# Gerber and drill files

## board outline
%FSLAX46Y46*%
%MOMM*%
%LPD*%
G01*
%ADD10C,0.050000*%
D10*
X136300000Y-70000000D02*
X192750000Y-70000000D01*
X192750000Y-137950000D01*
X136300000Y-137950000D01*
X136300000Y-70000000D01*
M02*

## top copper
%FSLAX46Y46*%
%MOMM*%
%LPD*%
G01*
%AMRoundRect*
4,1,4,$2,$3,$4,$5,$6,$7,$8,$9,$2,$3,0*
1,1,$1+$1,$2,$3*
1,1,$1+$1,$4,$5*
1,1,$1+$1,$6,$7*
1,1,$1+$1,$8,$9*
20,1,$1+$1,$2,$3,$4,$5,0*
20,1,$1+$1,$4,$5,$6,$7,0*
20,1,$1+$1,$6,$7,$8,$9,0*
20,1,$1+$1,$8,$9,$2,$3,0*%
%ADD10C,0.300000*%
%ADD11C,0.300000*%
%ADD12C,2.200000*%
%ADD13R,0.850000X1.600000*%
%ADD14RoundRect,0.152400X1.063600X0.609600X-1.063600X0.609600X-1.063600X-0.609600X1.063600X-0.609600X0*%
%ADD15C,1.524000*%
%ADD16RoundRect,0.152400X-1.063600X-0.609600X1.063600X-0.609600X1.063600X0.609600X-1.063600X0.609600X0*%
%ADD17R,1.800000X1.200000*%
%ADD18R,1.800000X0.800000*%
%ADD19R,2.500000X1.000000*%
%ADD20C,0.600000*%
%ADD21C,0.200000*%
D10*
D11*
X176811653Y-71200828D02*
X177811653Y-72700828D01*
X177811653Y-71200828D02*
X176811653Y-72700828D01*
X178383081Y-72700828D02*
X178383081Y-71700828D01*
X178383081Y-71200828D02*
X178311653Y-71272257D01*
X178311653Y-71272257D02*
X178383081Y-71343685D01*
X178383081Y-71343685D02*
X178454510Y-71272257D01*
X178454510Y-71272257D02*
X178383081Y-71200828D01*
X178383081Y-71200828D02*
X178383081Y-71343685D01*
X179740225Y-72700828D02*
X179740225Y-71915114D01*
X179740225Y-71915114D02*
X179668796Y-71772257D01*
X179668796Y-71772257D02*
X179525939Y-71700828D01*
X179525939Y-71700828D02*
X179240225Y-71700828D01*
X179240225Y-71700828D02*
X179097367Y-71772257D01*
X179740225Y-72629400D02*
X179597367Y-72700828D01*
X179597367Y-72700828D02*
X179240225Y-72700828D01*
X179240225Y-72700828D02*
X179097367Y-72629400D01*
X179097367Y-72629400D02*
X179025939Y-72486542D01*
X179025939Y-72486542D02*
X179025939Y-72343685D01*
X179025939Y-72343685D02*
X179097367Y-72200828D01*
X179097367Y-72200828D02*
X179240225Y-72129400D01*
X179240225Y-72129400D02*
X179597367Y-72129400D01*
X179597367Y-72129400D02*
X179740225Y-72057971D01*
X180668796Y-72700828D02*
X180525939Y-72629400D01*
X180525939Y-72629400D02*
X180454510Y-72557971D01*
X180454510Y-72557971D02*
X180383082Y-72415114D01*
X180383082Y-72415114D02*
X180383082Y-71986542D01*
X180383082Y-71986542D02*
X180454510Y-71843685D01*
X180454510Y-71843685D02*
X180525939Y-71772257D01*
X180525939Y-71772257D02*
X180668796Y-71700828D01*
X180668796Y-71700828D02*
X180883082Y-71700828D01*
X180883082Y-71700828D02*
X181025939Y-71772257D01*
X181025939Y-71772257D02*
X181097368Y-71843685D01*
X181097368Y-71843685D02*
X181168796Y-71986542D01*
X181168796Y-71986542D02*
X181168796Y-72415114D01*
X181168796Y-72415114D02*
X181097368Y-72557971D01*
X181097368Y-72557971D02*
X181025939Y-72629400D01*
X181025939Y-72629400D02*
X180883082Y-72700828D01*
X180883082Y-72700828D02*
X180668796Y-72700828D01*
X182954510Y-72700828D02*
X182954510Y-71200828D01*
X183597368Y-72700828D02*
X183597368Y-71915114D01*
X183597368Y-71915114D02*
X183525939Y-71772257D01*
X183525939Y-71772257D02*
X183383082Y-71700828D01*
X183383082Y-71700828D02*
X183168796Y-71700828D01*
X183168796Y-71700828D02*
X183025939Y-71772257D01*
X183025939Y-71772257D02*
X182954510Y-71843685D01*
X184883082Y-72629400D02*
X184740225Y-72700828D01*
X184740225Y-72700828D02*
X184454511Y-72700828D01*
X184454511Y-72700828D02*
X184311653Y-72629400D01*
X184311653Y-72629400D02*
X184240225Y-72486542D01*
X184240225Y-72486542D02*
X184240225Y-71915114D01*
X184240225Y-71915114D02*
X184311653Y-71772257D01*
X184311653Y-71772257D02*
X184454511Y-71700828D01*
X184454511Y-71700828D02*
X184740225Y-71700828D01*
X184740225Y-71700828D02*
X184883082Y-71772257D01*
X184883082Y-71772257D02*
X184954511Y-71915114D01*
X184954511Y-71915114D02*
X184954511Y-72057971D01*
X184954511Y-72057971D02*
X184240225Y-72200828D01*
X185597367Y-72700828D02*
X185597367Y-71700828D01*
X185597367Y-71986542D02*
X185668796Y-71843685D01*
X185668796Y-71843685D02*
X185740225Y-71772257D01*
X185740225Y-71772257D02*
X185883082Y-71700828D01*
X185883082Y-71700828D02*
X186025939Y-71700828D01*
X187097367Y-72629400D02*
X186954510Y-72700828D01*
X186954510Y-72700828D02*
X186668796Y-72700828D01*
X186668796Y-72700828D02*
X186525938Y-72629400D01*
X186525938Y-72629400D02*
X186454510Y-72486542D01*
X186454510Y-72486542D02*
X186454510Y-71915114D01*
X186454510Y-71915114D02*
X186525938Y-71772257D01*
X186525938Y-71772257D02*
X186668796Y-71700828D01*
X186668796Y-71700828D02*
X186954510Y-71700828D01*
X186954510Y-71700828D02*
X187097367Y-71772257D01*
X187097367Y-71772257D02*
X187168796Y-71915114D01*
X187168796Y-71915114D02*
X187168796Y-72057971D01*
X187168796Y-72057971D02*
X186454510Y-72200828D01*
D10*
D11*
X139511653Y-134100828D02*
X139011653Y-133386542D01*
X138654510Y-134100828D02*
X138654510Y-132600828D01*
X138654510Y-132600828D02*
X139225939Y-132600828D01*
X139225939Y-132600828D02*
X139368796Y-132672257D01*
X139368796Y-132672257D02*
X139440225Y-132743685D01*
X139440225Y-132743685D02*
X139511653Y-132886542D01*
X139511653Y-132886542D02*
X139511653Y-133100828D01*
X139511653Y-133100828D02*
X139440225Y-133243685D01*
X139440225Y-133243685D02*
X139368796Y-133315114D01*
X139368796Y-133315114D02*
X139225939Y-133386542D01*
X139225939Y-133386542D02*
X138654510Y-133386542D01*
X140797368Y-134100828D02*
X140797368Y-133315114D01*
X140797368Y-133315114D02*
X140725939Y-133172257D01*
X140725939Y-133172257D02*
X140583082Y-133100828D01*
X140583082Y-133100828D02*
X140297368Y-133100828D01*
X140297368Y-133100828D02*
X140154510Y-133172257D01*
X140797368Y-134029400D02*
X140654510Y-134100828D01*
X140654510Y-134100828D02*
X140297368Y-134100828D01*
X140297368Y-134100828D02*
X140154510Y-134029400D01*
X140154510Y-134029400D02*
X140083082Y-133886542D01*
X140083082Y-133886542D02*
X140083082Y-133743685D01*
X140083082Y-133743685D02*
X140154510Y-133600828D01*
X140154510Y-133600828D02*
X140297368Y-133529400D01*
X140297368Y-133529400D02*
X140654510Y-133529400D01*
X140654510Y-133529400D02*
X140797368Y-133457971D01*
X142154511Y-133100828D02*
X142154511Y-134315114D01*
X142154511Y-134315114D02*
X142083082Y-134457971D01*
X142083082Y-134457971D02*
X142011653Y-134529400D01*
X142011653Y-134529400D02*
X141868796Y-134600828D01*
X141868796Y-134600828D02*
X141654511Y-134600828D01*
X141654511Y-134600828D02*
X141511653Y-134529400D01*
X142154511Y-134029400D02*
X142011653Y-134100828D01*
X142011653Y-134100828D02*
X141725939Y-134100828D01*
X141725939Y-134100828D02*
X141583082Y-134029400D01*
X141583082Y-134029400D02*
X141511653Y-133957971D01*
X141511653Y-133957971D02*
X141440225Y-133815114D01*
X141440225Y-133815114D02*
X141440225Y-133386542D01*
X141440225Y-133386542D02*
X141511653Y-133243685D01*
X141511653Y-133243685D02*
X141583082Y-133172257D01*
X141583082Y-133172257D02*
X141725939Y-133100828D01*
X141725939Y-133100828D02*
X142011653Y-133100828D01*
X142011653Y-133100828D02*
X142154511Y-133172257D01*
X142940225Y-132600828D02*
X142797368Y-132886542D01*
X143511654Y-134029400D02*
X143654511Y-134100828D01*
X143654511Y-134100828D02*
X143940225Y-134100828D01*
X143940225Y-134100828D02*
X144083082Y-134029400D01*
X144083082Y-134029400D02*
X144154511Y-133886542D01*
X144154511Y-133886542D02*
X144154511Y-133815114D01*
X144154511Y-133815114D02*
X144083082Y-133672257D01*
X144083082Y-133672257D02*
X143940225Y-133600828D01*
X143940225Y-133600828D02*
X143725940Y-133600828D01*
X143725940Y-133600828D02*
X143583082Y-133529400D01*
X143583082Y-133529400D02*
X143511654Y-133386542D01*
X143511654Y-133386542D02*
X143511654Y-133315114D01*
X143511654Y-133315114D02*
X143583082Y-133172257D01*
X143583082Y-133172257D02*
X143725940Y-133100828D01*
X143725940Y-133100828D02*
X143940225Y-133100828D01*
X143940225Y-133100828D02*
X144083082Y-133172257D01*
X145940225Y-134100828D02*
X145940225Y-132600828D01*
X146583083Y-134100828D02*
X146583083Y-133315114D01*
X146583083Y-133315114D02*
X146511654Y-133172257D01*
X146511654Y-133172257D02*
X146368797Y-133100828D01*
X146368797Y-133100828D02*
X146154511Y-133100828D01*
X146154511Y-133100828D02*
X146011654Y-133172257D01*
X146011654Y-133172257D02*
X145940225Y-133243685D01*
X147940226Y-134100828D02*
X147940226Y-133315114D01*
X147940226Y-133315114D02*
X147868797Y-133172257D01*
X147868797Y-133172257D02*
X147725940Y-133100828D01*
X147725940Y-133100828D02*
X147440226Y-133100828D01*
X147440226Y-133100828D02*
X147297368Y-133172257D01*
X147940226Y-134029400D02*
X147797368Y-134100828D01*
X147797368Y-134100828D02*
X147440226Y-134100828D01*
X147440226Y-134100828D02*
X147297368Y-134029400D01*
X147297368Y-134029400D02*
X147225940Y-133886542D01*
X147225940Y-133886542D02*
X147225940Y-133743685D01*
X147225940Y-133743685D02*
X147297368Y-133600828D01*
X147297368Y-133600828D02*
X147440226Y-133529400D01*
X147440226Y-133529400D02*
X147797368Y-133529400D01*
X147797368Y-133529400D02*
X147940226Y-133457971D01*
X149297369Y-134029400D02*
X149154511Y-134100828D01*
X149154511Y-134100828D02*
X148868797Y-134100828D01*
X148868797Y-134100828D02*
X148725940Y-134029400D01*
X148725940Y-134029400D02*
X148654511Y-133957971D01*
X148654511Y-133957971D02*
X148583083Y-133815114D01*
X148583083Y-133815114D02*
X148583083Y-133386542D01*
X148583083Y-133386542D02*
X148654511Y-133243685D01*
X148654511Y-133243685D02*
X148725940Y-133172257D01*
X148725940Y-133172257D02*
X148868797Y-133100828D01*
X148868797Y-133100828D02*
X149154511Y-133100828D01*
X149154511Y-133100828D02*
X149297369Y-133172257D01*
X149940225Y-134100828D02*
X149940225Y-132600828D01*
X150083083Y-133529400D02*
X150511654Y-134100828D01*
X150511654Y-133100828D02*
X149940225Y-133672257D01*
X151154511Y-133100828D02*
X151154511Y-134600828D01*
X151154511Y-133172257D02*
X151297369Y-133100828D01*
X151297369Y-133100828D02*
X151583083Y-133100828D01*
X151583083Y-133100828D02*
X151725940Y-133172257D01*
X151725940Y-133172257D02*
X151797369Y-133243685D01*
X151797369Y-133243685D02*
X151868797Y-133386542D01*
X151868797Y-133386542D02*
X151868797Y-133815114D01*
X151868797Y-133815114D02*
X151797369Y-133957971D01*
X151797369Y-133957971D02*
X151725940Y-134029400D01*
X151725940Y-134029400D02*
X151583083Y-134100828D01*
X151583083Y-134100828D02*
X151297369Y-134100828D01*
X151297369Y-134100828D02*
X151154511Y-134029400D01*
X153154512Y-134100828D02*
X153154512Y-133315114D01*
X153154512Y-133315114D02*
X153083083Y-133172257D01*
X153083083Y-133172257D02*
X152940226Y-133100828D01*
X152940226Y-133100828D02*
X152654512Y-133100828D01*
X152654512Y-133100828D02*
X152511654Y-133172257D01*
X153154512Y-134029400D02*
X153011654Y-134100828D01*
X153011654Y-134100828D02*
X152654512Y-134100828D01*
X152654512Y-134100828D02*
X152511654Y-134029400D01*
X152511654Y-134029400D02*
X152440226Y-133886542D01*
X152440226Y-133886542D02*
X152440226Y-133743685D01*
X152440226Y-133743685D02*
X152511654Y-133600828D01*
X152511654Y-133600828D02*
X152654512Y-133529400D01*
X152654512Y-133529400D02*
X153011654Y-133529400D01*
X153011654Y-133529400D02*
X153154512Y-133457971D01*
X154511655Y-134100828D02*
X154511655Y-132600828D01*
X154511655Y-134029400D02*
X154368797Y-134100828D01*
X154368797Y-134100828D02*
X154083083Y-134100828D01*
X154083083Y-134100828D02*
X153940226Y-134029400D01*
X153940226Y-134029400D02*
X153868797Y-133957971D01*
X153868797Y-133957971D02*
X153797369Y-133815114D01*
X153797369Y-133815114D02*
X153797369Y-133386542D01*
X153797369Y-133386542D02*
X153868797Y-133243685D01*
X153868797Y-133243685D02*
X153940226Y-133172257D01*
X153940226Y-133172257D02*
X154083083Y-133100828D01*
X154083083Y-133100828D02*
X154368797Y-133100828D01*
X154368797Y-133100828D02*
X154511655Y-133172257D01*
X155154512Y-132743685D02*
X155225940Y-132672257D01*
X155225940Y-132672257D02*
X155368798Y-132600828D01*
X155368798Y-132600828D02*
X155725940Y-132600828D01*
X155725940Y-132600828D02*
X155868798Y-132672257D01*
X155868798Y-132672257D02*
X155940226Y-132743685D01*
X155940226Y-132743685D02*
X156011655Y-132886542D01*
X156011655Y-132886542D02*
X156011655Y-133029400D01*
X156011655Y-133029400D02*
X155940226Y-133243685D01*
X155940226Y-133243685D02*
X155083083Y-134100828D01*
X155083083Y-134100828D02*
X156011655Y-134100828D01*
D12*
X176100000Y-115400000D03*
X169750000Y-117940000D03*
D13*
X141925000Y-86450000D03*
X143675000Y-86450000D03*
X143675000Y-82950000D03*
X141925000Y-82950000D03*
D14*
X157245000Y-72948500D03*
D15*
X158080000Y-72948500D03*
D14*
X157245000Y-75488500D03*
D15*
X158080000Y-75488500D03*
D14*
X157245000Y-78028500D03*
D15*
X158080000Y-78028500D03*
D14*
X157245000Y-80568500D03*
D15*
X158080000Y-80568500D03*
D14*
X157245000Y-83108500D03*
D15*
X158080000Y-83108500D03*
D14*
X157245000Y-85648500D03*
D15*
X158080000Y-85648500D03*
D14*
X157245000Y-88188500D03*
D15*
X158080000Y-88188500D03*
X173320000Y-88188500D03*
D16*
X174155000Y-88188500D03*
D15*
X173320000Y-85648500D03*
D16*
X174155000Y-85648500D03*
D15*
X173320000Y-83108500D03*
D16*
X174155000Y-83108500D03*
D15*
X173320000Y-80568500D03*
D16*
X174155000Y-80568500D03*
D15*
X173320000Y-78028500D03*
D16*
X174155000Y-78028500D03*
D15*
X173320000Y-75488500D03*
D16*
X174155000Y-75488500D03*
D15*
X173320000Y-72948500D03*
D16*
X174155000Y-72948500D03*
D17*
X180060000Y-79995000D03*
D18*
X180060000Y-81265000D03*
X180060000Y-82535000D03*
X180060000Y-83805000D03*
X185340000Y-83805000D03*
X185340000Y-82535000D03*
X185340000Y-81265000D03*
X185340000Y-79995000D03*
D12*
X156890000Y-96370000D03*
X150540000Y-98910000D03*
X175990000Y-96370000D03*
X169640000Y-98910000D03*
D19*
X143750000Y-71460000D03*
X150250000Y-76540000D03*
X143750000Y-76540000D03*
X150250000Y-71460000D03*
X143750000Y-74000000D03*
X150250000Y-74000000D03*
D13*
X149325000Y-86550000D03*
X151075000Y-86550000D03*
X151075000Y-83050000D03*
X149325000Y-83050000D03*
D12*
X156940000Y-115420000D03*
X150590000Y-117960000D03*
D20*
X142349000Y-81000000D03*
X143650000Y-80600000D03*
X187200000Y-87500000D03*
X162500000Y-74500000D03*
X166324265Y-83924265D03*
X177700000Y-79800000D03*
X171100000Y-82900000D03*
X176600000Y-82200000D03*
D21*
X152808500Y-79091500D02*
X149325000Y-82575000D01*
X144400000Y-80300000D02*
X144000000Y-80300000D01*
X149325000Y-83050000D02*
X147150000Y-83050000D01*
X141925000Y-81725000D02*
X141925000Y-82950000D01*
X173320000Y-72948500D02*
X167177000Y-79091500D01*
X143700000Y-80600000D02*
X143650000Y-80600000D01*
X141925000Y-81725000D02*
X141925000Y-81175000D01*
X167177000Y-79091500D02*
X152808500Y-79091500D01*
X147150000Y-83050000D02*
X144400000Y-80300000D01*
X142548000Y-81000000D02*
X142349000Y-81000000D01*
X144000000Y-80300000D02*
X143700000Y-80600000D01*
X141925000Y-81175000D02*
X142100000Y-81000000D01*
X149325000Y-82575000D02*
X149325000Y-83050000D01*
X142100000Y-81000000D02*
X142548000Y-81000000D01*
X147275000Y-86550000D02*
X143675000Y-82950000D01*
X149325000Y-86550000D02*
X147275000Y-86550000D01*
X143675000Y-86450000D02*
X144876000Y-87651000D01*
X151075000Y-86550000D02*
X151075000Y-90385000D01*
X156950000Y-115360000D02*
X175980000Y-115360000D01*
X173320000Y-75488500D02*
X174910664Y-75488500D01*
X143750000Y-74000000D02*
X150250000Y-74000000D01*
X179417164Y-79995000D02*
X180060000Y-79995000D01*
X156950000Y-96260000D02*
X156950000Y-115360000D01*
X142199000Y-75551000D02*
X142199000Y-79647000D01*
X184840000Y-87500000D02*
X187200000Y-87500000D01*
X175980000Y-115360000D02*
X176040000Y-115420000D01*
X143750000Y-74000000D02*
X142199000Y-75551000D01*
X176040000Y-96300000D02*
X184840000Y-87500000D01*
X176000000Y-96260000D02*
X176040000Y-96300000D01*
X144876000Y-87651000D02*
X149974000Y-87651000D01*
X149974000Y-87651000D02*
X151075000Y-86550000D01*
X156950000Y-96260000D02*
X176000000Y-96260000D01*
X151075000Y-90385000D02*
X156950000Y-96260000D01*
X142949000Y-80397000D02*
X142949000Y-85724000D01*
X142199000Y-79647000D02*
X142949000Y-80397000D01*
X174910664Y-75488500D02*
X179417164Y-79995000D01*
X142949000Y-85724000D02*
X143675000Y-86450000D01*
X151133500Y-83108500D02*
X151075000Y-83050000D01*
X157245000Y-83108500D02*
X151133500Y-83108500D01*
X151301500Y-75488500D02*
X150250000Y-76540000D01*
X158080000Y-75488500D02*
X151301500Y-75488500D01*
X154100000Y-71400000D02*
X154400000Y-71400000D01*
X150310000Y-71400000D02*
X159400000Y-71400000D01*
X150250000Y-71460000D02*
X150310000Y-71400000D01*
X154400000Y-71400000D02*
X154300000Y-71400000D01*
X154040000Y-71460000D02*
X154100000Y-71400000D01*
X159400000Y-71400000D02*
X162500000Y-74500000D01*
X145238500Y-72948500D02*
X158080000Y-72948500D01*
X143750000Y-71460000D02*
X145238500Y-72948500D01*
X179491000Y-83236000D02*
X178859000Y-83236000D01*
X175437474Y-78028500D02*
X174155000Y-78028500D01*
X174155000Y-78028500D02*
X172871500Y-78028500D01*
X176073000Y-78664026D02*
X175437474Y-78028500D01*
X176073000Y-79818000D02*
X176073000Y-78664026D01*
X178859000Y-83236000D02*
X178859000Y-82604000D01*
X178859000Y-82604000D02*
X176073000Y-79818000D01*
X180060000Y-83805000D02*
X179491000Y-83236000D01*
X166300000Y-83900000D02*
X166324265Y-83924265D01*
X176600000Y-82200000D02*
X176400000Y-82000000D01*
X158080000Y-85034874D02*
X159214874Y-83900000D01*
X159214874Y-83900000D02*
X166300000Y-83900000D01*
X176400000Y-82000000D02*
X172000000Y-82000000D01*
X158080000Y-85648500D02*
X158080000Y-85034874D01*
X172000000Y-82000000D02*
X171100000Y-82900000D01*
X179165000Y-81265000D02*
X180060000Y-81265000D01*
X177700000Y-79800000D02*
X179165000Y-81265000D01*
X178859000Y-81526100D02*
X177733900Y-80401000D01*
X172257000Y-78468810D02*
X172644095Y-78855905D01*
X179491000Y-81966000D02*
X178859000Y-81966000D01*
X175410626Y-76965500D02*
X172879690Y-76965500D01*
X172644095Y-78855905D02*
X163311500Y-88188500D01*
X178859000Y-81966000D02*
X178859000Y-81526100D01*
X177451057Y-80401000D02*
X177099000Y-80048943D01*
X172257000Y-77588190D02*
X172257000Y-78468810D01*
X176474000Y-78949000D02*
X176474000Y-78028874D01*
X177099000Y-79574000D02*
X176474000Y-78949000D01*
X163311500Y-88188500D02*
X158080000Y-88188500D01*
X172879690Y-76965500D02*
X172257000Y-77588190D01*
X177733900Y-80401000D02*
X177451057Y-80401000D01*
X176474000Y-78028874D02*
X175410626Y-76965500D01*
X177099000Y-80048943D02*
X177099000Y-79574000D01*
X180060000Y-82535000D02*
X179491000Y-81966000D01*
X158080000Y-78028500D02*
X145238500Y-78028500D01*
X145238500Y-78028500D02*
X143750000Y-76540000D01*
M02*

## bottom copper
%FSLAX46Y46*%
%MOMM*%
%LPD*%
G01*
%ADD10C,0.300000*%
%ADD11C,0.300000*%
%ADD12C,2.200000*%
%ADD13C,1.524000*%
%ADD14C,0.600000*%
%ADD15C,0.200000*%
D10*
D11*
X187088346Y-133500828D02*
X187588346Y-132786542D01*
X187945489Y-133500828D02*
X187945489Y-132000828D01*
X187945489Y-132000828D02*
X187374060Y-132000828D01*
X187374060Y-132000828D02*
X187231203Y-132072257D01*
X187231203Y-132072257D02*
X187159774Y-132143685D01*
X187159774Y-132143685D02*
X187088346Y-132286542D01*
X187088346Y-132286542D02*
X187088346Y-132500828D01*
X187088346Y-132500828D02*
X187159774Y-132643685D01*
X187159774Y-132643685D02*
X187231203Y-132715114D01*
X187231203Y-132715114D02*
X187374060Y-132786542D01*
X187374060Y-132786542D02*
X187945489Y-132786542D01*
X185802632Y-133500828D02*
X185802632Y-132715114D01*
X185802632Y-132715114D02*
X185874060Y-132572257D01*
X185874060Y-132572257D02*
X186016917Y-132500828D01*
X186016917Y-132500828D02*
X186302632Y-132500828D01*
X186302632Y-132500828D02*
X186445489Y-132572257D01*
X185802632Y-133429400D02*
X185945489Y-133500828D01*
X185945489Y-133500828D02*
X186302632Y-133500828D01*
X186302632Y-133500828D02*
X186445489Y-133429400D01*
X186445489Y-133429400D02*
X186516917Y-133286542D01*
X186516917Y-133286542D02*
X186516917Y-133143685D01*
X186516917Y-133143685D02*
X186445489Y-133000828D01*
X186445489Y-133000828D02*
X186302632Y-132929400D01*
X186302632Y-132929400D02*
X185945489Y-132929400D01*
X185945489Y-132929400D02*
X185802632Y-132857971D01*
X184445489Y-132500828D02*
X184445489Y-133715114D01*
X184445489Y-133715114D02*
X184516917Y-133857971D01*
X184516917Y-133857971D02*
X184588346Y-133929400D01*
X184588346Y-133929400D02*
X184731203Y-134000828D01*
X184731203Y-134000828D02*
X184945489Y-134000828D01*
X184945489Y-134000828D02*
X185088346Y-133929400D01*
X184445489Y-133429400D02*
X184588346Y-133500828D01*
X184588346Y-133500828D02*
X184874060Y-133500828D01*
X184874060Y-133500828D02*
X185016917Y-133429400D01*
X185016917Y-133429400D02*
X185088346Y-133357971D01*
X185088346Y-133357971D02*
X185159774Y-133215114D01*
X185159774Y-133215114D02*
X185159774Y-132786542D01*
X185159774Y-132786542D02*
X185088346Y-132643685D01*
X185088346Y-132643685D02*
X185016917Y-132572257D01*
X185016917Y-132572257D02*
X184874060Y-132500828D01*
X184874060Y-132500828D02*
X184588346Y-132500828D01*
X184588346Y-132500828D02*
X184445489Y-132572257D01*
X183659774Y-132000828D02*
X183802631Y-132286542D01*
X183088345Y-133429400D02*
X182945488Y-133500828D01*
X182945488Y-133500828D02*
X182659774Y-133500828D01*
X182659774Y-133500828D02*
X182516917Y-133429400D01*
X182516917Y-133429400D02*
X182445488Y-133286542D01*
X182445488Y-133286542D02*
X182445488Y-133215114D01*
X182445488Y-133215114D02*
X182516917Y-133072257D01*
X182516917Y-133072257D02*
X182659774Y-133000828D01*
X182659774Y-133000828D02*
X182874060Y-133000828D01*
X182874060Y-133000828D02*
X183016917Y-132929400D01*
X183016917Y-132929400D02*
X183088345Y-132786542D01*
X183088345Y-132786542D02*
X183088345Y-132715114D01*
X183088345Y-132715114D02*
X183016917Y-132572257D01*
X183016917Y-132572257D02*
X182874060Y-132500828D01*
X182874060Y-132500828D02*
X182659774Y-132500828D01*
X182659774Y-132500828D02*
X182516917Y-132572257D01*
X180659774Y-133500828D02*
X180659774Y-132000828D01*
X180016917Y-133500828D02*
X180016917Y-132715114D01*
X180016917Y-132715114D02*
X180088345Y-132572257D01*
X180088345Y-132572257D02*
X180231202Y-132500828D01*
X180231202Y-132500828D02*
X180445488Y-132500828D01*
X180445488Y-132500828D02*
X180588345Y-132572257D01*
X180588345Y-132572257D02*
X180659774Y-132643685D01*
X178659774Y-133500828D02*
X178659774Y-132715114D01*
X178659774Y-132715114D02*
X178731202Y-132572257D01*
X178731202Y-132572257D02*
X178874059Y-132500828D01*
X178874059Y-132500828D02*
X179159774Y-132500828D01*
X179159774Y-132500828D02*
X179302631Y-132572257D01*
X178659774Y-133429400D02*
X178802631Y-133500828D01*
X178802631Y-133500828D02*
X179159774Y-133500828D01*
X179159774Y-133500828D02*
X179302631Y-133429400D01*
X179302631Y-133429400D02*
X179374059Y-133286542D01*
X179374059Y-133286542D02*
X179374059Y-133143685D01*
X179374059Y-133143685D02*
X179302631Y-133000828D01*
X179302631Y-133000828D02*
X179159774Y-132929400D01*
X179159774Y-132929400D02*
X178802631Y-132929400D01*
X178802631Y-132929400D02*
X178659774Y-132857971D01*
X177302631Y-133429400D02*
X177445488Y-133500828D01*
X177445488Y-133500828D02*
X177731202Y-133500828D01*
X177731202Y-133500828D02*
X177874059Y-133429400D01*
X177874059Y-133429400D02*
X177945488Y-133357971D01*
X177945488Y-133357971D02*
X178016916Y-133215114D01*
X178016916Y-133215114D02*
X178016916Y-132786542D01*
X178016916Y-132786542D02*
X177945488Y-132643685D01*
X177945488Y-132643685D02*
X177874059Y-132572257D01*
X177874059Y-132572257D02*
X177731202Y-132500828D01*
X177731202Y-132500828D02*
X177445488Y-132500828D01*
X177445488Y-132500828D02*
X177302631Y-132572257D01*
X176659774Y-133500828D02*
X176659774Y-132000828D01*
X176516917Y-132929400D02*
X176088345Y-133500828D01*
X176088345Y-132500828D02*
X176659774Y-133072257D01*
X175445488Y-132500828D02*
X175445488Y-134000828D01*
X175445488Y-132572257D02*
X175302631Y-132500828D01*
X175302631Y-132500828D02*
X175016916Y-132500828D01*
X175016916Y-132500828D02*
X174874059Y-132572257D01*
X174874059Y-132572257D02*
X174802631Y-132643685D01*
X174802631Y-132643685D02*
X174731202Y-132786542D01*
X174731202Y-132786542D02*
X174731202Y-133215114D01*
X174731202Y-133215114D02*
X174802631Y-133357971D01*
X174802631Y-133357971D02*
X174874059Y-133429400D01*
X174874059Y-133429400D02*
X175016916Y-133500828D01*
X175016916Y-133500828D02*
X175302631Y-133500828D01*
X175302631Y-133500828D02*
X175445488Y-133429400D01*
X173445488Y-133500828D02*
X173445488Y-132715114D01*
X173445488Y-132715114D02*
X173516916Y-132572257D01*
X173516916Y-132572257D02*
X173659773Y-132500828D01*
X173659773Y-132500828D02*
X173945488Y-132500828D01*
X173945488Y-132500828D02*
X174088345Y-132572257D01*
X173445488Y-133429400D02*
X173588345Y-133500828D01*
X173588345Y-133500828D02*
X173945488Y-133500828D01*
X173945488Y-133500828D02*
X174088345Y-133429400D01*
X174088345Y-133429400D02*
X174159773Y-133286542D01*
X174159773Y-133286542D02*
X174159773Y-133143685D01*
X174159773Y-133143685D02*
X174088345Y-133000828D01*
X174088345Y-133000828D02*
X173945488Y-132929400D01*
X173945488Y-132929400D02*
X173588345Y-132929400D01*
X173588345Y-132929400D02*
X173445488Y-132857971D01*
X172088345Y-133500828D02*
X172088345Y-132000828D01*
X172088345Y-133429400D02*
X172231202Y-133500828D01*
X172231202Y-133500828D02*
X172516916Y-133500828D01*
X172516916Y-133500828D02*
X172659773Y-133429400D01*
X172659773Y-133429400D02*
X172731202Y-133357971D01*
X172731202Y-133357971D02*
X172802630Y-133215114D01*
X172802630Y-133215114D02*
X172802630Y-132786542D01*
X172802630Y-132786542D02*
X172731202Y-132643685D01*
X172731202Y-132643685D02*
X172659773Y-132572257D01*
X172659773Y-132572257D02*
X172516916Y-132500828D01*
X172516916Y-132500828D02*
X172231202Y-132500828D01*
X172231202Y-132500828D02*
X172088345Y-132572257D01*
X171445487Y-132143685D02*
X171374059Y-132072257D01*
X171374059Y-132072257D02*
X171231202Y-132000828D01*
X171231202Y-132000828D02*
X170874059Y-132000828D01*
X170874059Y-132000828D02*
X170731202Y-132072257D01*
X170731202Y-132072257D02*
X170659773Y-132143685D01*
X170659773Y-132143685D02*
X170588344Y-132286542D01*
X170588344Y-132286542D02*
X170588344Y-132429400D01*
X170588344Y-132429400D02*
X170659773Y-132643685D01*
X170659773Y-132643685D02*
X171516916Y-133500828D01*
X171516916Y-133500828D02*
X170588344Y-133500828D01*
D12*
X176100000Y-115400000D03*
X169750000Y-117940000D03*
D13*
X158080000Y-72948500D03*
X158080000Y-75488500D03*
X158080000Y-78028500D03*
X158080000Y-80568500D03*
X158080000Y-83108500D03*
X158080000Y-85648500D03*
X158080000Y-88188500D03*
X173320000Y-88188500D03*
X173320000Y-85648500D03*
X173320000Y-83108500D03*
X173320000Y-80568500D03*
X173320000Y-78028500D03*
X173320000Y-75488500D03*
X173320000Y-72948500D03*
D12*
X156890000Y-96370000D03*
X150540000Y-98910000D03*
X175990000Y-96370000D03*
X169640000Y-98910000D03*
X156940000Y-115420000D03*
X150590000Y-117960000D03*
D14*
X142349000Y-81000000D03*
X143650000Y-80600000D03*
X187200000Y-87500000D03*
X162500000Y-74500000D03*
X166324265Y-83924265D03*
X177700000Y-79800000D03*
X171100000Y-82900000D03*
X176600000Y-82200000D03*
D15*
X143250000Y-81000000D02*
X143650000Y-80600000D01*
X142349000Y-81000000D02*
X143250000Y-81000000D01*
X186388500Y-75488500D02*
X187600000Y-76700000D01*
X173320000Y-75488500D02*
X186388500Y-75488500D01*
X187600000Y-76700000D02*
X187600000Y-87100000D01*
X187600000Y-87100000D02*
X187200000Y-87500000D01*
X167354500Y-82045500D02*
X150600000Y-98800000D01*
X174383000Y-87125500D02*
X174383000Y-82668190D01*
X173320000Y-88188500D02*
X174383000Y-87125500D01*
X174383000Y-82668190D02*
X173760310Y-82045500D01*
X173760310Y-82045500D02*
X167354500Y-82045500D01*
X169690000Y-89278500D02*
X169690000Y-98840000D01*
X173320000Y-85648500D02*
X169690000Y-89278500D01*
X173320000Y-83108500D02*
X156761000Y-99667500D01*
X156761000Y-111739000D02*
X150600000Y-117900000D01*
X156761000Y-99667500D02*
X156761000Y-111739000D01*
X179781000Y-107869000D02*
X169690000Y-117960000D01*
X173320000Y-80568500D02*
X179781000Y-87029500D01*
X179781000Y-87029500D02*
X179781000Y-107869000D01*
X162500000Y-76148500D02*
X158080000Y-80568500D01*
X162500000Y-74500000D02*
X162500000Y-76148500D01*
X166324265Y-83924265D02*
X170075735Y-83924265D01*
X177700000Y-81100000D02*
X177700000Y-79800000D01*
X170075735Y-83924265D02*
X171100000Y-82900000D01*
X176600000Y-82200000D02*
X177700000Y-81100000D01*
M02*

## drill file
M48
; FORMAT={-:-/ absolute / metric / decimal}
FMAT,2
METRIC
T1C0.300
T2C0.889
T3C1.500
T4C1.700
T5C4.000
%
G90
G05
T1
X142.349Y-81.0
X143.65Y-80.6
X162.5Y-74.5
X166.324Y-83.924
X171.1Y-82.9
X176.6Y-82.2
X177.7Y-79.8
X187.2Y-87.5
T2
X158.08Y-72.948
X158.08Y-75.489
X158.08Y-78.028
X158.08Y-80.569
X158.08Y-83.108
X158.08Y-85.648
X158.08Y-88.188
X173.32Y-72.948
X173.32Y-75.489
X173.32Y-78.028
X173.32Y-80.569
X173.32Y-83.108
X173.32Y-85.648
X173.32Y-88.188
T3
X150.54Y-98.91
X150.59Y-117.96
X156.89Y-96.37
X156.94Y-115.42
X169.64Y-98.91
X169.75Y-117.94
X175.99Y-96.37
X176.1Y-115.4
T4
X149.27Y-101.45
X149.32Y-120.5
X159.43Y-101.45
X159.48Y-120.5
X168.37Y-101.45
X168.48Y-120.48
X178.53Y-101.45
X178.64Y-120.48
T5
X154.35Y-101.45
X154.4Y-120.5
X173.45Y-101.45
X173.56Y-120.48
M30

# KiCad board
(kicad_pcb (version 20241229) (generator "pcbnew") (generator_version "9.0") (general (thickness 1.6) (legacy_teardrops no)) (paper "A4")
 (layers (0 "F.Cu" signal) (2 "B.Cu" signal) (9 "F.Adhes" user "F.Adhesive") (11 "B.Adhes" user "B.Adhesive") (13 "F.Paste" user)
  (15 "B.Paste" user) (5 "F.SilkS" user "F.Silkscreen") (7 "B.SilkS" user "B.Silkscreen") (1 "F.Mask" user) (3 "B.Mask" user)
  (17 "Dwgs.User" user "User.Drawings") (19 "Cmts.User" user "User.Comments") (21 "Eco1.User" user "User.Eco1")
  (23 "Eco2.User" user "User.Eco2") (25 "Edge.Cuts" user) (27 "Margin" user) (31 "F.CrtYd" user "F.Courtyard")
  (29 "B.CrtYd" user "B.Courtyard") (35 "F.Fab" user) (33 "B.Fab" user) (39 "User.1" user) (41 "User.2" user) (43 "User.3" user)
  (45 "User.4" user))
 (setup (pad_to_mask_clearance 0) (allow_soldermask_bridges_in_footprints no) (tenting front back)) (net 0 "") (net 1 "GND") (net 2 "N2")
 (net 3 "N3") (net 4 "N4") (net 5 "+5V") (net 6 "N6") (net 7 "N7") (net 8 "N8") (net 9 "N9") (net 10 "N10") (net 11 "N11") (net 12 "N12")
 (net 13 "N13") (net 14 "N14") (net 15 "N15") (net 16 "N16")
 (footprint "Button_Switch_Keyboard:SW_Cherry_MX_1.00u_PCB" (layer "F.Cu") (at 176.1 115.4)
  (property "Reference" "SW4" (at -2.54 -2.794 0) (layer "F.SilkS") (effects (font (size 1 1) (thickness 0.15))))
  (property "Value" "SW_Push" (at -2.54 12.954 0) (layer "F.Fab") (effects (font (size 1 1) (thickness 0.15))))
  (pad "" np_thru_hole circle (at -7.62 5.08) (size 1.7 1.7) (drill 1.7) (layers "*.Cu" "*.Mask"))
  (pad "" np_thru_hole circle (at -2.54 5.08) (size 4 4) (drill 4) (layers "*.Cu" "*.Mask"))
  (pad "" np_thru_hole circle (at 2.54 5.08) (size 1.7 1.7) (drill 1.7) (layers "*.Cu" "*.Mask"))
  (pad "1" thru_hole circle (at 0 0) (size 2.2 2.2) (drill 1.5) (layers "*.Cu" "*.Mask") (remove_unused_layers no) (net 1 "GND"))
  (pad "2" thru_hole circle (at -6.35 2.54) (size 2.2 2.2) (drill 1.5) (layers "*.Cu" "*.Mask") (remove_unused_layers no) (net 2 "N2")))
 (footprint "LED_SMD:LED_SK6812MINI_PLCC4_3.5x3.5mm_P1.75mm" (layer "F.Cu") (at 142.8 84.7 90)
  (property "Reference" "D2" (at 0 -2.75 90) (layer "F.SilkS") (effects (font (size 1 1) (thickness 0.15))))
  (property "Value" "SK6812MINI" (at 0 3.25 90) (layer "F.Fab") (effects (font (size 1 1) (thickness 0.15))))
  (pad "1" smd rect (at -1.75 -0.875 90) (size 1.6 0.85) (layers "F.Cu" "F.Mask" "F.Paste") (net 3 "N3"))
  (pad "2" smd rect (at -1.75 0.875 90) (size 1.6 0.85) (layers "F.Cu" "F.Mask" "F.Paste") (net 1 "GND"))
  (pad "3" smd rect (at 1.75 0.875 90) (size 1.6 0.85) (layers "F.Cu" "F.Mask" "F.Paste") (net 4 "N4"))
  (pad "4" smd rect (at 1.75 -0.875 90) (size 1.6 0.85) (layers "F.Cu" "F.Mask" "F.Paste") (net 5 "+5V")))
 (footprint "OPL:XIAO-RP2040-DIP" (layer "F.Cu") (at 165.7 80.5685)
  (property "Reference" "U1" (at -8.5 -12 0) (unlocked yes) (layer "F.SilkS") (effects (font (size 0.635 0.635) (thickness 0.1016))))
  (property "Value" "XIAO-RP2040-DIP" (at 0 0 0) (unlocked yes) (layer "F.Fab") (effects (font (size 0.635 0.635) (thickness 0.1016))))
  (pad "1" smd roundrect (at -8.455 -7.62 180) (size 2.432 1.524) (layers "F.Cu" "F.Mask") (roundrect_rratio 0.1) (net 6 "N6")
   (thermal_bridge_angle 45))
  (pad "1" thru_hole circle (at -7.62 -7.62 180) (size 1.524 1.524) (drill 0.889) (layers "*.Cu" "*.Mask") (remove_unused_layers no)
   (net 6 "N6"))
  (pad "2" smd roundrect (at -8.455 -5.08 180) (size 2.432 1.524) (layers "F.Cu" "F.Mask") (roundrect_rratio 0.1) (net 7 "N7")
   (thermal_bridge_angle 45))
  (pad "2" thru_hole circle (at -7.62 -5.08 180) (size 1.524 1.524) (drill 0.889) (layers "*.Cu" "*.Mask") (remove_unused_layers no)
   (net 7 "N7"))
  (pad "3" smd roundrect (at -8.455 -2.54 180) (size 2.432 1.524) (layers "F.Cu" "F.Mask") (roundrect_rratio 0.1) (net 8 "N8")
   (thermal_bridge_angle 45))
  (pad "3" thru_hole circle (at -7.62 -2.54 180) (size 1.524 1.524) (drill 0.889) (layers "*.Cu" "*.Mask") (remove_unused_layers no)
   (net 8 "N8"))
  (pad "4" smd roundrect (at -8.455 0 180) (size 2.432 1.524) (layers "F.Cu" "F.Mask") (roundrect_rratio 0.1) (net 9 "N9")
   (thermal_bridge_angle 45))
  (pad "4" thru_hole circle (at -7.62 0 180) (size 1.524 1.524) (drill 0.889) (layers "*.Cu" "*.Mask") (remove_unused_layers no)
   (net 9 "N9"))
  (pad "5" smd roundrect (at -8.455 2.54 180) (size 2.432 1.524) (layers "F.Cu" "F.Mask") (roundrect_rratio 0.1) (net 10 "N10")
   (thermal_bridge_angle 45))
  (pad "5" thru_hole circle (at -7.62 2.54 180) (size 1.524 1.524) (drill 0.889) (layers "*.Cu" "*.Mask") (remove_unused_layers no)
   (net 10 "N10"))
  (pad "6" smd roundrect (at -8.455 5.08 180) (size 2.432 1.524) (layers "F.Cu" "F.Mask") (roundrect_rratio 0.1) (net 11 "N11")
   (thermal_bridge_angle 45))
  (pad "6" thru_hole circle (at -7.62 5.08 180) (size 1.524 1.524) (drill 0.889) (layers "*.Cu" "*.Mask") (remove_unused_layers no)
   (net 11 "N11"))
  (pad "7" smd roundrect (at -8.455 7.62 180) (size 2.432 1.524) (layers "F.Cu" "F.Mask") (roundrect_rratio 0.1) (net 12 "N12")
   (thermal_bridge_angle 45))
  (pad "7" thru_hole circle (at -7.62 7.62 180) (size 1.524 1.524) (drill 0.889) (layers "*.Cu" "*.Mask") (remove_unused_layers no)
   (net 12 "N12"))
  (pad "8" thru_hole circle (at 7.62 7.62) (size 1.524 1.524) (drill 0.889) (layers "*.Cu" "*.Mask") (remove_unused_layers no)
   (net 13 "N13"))
  (pad "8" smd roundrect (at 8.455 7.62) (size 2.432 1.524) (layers "F.Cu" "F.Mask") (roundrect_rratio 0.1) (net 13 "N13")
   (thermal_bridge_angle 45))
  (pad "9" thru_hole circle (at 7.62 5.08) (size 1.524 1.524) (drill 0.889) (layers "*.Cu" "*.Mask") (remove_unused_layers no)
   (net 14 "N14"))
  (pad "9" smd roundrect (at 8.455 5.08) (size 2.432 1.524) (layers "F.Cu" "F.Mask") (roundrect_rratio 0.1) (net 14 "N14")
   (thermal_bridge_angle 45))
  (pad "10" thru_hole circle (at 7.62 2.54) (size 1.524 1.524) (drill 0.889) (layers "*.Cu" "*.Mask") (remove_unused_layers no)
   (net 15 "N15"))
  (pad "10" smd roundrect (at 8.455 2.54) (size 2.432 1.524) (layers "F.Cu" "F.Mask") (roundrect_rratio 0.1) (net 15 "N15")
   (thermal_bridge_angle 45))
  (pad "11" thru_hole circle (at 7.62 0) (size 1.524 1.524) (drill 0.889) (layers "*.Cu" "*.Mask") (remove_unused_layers no) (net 2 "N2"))
  (pad "11" smd roundrect (at 8.455 0) (size 2.432 1.524) (layers "F.Cu" "F.Mask") (roundrect_rratio 0.1) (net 2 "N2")
   (thermal_bridge_angle 45))
  (pad "12" thru_hole circle (at 7.62 -2.54) (size 1.524 1.524) (drill 0.889) (layers "*.Cu" "*.Mask") (remove_unused_layers no)
   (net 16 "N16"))
  (pad "12" smd roundrect (at 8.455 -2.54) (size 2.432 1.524) (layers "F.Cu" "F.Mask") (roundrect_rratio 0.1) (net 16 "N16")
   (thermal_bridge_angle 45))
  (pad "13" thru_hole circle (at 7.62 -5.08) (size 1.524 1.524) (drill 0.889) (layers "*.Cu" "*.Mask") (remove_unused_layers no)
   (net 1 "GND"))
  (pad "13" smd roundrect (at 8.455 -5.08) (size 2.432 1.524) (layers "F.Cu" "F.Mask") (roundrect_rratio 0.1) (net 1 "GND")
   (thermal_bridge_angle 45))
  (pad "14" thru_hole circle (at 7.62 -7.62) (size 1.524 1.524) (drill 0.889) (layers "*.Cu" "*.Mask") (remove_unused_layers no)
   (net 5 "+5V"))
  (pad "14" smd roundrect (at 8.455 -7.62) (size 2.432 1.524) (layers "F.Cu" "F.Mask") (roundrect_rratio 0.1) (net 5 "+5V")
   (thermal_bridge_angle 45)))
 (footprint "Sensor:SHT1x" (layer "F.Cu") (at 182.7 81.9)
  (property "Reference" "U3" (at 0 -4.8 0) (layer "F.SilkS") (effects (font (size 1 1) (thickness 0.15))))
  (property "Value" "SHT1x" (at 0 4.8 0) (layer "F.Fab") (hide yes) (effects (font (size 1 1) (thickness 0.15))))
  (pad "1" smd rect (at -2.64 -1.905) (size 1.8 1.2) (layers "F.Cu" "F.Mask" "F.Paste") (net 1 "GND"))
  (pad "2" smd rect (at -2.64 -0.635) (size 1.8 0.8) (layers "F.Cu" "F.Mask" "F.Paste") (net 11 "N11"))
  (pad "3" smd rect (at -2.64 0.635) (size 1.8 0.8) (layers "F.Cu" "F.Mask" "F.Paste") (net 12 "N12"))
  (pad "4" smd rect (at -2.64 1.905) (size 1.8 0.8) (layers "F.Cu" "F.Mask" "F.Paste") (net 16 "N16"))
  (pad "5" smd rect (at 2.64 1.905) (size 1.8 0.8) (layers "F.Cu" "F.Mask" "F.Paste"))
  (pad "6" smd rect (at 2.64 0.635) (size 1.8 0.8) (layers "F.Cu" "F.Mask" "F.Paste"))
  (pad "7" smd rect (at 2.64 -0.635) (size 1.8 0.8) (layers "F.Cu" "F.Mask" "F.Paste"))
  (pad "8" smd rect (at 2.64 -1.905) (size 1.8 0.8) (layers "F.Cu" "F.Mask" "F.Paste"))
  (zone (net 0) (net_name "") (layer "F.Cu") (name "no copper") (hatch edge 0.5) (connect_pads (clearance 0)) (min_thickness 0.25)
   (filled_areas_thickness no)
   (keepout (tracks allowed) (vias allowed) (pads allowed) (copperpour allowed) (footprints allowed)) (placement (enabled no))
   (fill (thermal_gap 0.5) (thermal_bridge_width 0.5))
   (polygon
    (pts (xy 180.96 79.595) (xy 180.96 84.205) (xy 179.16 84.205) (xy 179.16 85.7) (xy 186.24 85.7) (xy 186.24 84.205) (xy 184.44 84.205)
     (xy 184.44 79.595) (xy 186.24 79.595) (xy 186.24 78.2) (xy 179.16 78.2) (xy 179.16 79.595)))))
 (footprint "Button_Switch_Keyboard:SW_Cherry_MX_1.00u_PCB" (layer "F.Cu") (at 156.89 96.37)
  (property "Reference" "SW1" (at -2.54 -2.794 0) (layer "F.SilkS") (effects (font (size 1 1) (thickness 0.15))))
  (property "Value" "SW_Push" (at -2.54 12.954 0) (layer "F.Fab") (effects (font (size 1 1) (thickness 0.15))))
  (pad "" np_thru_hole circle (at -7.62 5.08) (size 1.7 1.7) (drill 1.7) (layers "*.Cu" "*.Mask"))
  (pad "" np_thru_hole circle (at -2.54 5.08) (size 4 4) (drill 4) (layers "*.Cu" "*.Mask"))
  (pad "" np_thru_hole circle (at 2.54 5.08) (size 1.7 1.7) (drill 1.7) (layers "*.Cu" "*.Mask"))
  (pad "1" thru_hole circle (at 0 0) (size 2.2 2.2) (drill 1.5) (layers "*.Cu" "*.Mask") (remove_unused_layers no) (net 1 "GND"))
  (pad "2" thru_hole circle (at -6.35 2.54) (size 2.2 2.2) (drill 1.5) (layers "*.Cu" "*.Mask") (remove_unused_layers no) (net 13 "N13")))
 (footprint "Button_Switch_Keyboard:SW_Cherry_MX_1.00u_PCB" (layer "F.Cu") (at 175.99 96.37)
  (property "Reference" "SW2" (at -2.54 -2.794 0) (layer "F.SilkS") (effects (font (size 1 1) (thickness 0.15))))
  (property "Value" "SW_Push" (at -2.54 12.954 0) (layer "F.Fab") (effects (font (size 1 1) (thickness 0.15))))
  (pad "" np_thru_hole circle (at -7.62 5.08) (size 1.7 1.7) (drill 1.7) (layers "*.Cu" "*.Mask"))
  (pad "" np_thru_hole circle (at -2.54 5.08) (size 4 4) (drill 4) (layers "*.Cu" "*.Mask"))
  (pad "" np_thru_hole circle (at 2.54 5.08) (size 1.7 1.7) (drill 1.7) (layers "*.Cu" "*.Mask"))
  (pad "1" thru_hole circle (at 0 0) (size 2.2 2.2) (drill 1.5) (layers "*.Cu" "*.Mask") (remove_unused_layers no) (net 1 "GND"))
  (pad "2" thru_hole circle (at -6.35 2.54) (size 2.2 2.2) (drill 1.5) (layers "*.Cu" "*.Mask") (remove_unused_layers no) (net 14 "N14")))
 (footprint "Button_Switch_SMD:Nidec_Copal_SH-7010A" (layer "F.Cu") (at 147 74)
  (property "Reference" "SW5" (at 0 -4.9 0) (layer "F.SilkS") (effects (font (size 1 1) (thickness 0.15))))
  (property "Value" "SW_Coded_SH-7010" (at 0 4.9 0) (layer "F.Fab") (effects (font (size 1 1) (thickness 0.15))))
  (pad "1" smd rect (at -3.25 -2.54) (size 2.5 1) (layers "F.Cu" "F.Mask" "F.Paste") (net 6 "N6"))
  (pad "2" smd rect (at 3.25 2.54) (size 2.5 1) (layers "F.Cu" "F.Mask" "F.Paste") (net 7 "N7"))
  (pad "4" smd rect (at -3.25 2.54) (size 2.5 1) (layers "F.Cu" "F.Mask" "F.Paste") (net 8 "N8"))
  (pad "8" smd rect (at 3.25 -2.54) (size 2.5 1) (layers "F.Cu" "F.Mask" "F.Paste") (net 9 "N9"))
  (pad "C" smd rect (at -3.25 0) (size 2.5 1) (layers "F.Cu" "F.Mask" "F.Paste") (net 1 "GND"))
  (pad "C" smd rect (at 3.25 0) (size 2.5 1) (layers "F.Cu" "F.Mask" "F.Paste") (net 1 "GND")))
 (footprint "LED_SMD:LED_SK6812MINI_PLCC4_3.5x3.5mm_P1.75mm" (layer "F.Cu") (at 150.2 84.8 90)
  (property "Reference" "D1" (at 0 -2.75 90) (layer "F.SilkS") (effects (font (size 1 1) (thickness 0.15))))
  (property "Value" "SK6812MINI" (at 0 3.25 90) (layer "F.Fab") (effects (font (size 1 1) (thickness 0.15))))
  (pad "1" smd rect (at -1.75 -0.875 90) (size 1.6 0.85) (layers "F.Cu" "F.Mask" "F.Paste") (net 4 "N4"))
  (pad "2" smd rect (at -1.75 0.875 90) (size 1.6 0.85) (layers "F.Cu" "F.Mask" "F.Paste") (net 1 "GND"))
  (pad "3" smd rect (at 1.75 0.875 90) (size 1.6 0.85) (layers "F.Cu" "F.Mask" "F.Paste") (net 10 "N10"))
  (pad "4" smd rect (at 1.75 -0.875 90) (size 1.6 0.85) (layers "F.Cu" "F.Mask" "F.Paste") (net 5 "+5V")))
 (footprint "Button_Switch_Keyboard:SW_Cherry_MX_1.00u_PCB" (layer "F.Cu") (at 156.94 115.42)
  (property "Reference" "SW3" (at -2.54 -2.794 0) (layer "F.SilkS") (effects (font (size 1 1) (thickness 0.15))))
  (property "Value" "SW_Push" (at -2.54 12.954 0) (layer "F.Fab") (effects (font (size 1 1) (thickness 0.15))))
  (pad "" np_thru_hole circle (at -7.62 5.08) (size 1.7 1.7) (drill 1.7) (layers "*.Cu" "*.Mask"))
  (pad "" np_thru_hole circle (at -2.54 5.08) (size 4 4) (drill 4) (layers "*.Cu" "*.Mask"))
  (pad "" np_thru_hole circle (at 2.54 5.08) (size 1.7 1.7) (drill 1.7) (layers "*.Cu" "*.Mask"))
  (pad "1" thru_hole circle (at 0 0) (size 2.2 2.2) (drill 1.5) (layers "*.Cu" "*.Mask") (remove_unused_layers no) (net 1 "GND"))
  (pad "2" thru_hole circle (at -6.35 2.54) (size 2.2 2.2) (drill 1.5) (layers "*.Cu" "*.Mask") (remove_unused_layers no) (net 15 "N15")))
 (gr_rect (start 136.3 70) (end 192.75 137.95) (stroke (width 0.05) (type default)) (fill no) (layer "Edge.Cuts"))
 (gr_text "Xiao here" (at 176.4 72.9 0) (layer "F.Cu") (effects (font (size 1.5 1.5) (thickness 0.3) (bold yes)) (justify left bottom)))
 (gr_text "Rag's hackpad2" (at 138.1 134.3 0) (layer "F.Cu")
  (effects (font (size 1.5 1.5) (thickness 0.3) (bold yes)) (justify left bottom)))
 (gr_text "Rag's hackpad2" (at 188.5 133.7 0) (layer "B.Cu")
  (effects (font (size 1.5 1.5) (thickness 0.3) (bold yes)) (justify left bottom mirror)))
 (segment (start 152.8085 79.0915) (end 149.325 82.575) (width 0.2) (layer "F.Cu") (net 5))
 (segment (start 144.4 80.3) (end 144 80.3) (width 0.2) (layer "F.Cu") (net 5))
 (segment (start 149.325 83.05) (end 147.15 83.05) (width 0.2) (layer "F.Cu") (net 5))
 (segment (start 141.925 81.725) (end 141.925 82.95) (width 0.2) (layer "F.Cu") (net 5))
 (segment (start 173.32 72.9485) (end 167.177 79.0915) (width 0.2) (layer "F.Cu") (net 5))
 (segment (start 143.7 80.6) (end 143.65 80.6) (width 0.2) (layer "F.Cu") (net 5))
 (segment (start 141.925 81.725) (end 141.925 81.175) (width 0.2) (layer "F.Cu") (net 5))
 (segment (start 167.177 79.0915) (end 152.8085 79.0915) (width 0.2) (layer "F.Cu") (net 5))
 (segment (start 147.15 83.05) (end 144.4 80.3) (width 0.2) (layer "F.Cu") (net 5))
 (segment (start 142.548 81) (end 142.349 81) (width 0.2) (layer "F.Cu") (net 5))
 (segment (start 144 80.3) (end 143.7 80.6) (width 0.2) (layer "F.Cu") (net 5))
 (segment (start 141.925 81.175) (end 142.1 81) (width 0.2) (layer "F.Cu") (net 5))
 (segment (start 149.325 82.575) (end 149.325 83.05) (width 0.2) (layer "F.Cu") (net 5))
 (segment (start 142.1 81) (end 142.548 81) (width 0.2) (layer "F.Cu") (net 5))
 (via (at 142.349 81) (size 0.6) (drill 0.3) (layers "F.Cu" "B.Cu") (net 5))
 (via (at 143.65 80.6) (size 0.6) (drill 0.3) (layers "F.Cu" "B.Cu") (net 5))
 (segment (start 143.25 81) (end 143.65 80.6) (width 0.2) (layer "B.Cu") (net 5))
 (segment (start 142.349 81) (end 143.25 81) (width 0.2) (layer "B.Cu") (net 5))
 (segment (start 147.275 86.55) (end 143.675 82.95) (width 0.2) (layer "F.Cu") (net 4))
 (segment (start 149.325 86.55) (end 147.275 86.55) (width 0.2) (layer "F.Cu") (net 4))
 (segment (start 143.675 86.45) (end 144.876 87.651) (width 0.2) (layer "F.Cu") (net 1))
 (segment (start 151.075 86.55) (end 151.075 90.385) (width 0.2) (layer "F.Cu") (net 1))
 (segment (start 156.95 115.36) (end 175.98 115.36) (width 0.2) (layer "F.Cu") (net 1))
 (segment (start 173.32 75.4885) (end 174.910664 75.4885) (width 0.2) (layer "F.Cu") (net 1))
 (segment (start 143.75 74) (end 150.25 74) (width 0.2) (layer "F.Cu") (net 1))
 (segment (start 179.417164 79.995) (end 180.06 79.995) (width 0.2) (layer "F.Cu") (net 1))
 (segment (start 156.95 96.26) (end 156.95 115.36) (width 0.2) (layer "F.Cu") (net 1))
 (segment (start 142.199 75.551) (end 142.199 79.647) (width 0.2) (layer "F.Cu") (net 1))
 (segment (start 184.84 87.5) (end 187.2 87.5) (width 0.2) (layer "F.Cu") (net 1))
 (segment (start 175.98 115.36) (end 176.04 115.42) (width 0.2) (layer "F.Cu") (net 1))
 (segment (start 143.75 74) (end 142.199 75.551) (width 0.2) (layer "F.Cu") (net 1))
 (segment (start 176.04 96.3) (end 184.84 87.5) (width 0.2) (layer "F.Cu") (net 1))
 (segment (start 176 96.26) (end 176.04 96.3) (width 0.2) (layer "F.Cu") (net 1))
 (segment (start 144.876 87.651) (end 149.974 87.651) (width 0.2) (layer "F.Cu") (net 1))
 (segment (start 149.974 87.651) (end 151.075 86.55) (width 0.2) (layer "F.Cu") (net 1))
 (segment (start 156.95 96.26) (end 176 96.26) (width 0.2) (layer "F.Cu") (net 1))
 (segment (start 151.075 90.385) (end 156.95 96.26) (width 0.2) (layer "F.Cu") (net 1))
 (segment (start 142.949 80.397) (end 142.949 85.724) (width 0.2) (layer "F.Cu") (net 1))
 (segment (start 142.199 79.647) (end 142.949 80.397) (width 0.2) (layer "F.Cu") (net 1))
 (segment (start 174.910664 75.4885) (end 179.417164 79.995) (width 0.2) (layer "F.Cu") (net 1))
 (segment (start 142.949 85.724) (end 143.675 86.45) (width 0.2) (layer "F.Cu") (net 1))
 (via (at 187.2 87.5) (size 0.6) (drill 0.3) (layers "F.Cu" "B.Cu") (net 1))
 (segment (start 186.3885 75.4885) (end 187.6 76.7) (width 0.2) (layer "B.Cu") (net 1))
 (segment (start 173.32 75.4885) (end 186.3885 75.4885) (width 0.2) (layer "B.Cu") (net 1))
 (segment (start 187.6 76.7) (end 187.6 87.1) (width 0.2) (layer "B.Cu") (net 1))
 (segment (start 187.6 87.1) (end 187.2 87.5) (width 0.2) (layer "B.Cu") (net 1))
 (segment (start 151.1335 83.1085) (end 151.075 83.05) (width 0.2) (layer "F.Cu") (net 10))
 (segment (start 157.245 83.1085) (end 151.1335 83.1085) (width 0.2) (layer "F.Cu") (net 10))
 (segment (start 167.3545 82.0455) (end 150.6 98.8) (width 0.2) (layer "B.Cu") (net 13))
 (segment (start 174.383 87.1255) (end 174.383 82.66819) (width 0.2) (layer "B.Cu") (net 13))
 (segment (start 173.32 88.1885) (end 174.383 87.1255) (width 0.2) (layer "B.Cu") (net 13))
 (segment (start 174.383 82.66819) (end 173.76031 82.0455) (width 0.2) (layer "B.Cu") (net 13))
 (segment (start 173.76031 82.0455) (end 167.3545 82.0455) (width 0.2) (layer "B.Cu") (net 13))
 (segment (start 169.69 89.2785) (end 169.69 98.84) (width 0.2) (layer "B.Cu") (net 14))
 (segment (start 173.32 85.6485) (end 169.69 89.2785) (width 0.2) (layer "B.Cu") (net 14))
 (segment (start 173.32 83.1085) (end 156.761 99.6675) (width 0.2) (layer "B.Cu") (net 15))
 (segment (start 156.761 111.739) (end 150.6 117.9) (width 0.2) (layer "B.Cu") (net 15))
 (segment (start 156.761 99.6675) (end 156.761 111.739) (width 0.2) (layer "B.Cu") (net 15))
 (segment (start 179.781 107.869) (end 169.69 117.96) (width 0.2) (layer "B.Cu") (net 2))
 (segment (start 173.32 80.5685) (end 179.781 87.0295) (width 0.2) (layer "B.Cu") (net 2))
 (segment (start 179.781 87.0295) (end 179.781 107.869) (width 0.2) (layer "B.Cu") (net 2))
 (segment (start 151.3015 75.4885) (end 150.25 76.54) (width 0.2) (layer "F.Cu") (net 7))
 (segment (start 158.08 75.4885) (end 151.3015 75.4885) (width 0.2) (layer "F.Cu") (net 7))
 (segment (start 154.1 71.4) (end 154.4 71.4) (width 0.2) (layer "F.Cu") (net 9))
 (segment (start 150.31 71.4) (end 159.4 71.4) (width 0.2) (layer "F.Cu") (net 9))
 (segment (start 150.25 71.46) (end 150.31 71.4) (width 0.2) (layer "F.Cu") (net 9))
 (segment (start 154.4 71.4) (end 154.3 71.4) (width 0.2) (layer "F.Cu") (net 9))
 (segment (start 154.04 71.46) (end 154.1 71.4) (width 0.2) (layer "F.Cu") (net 9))
 (segment (start 159.4 71.4) (end 162.5 74.5) (width 0.2) (layer "F.Cu") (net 9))
 (via (at 162.5 74.5) (size 0.6) (drill 0.3) (layers "F.Cu" "B.Cu") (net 9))
 (segment (start 162.5 76.1485) (end 158.08 80.5685) (width 0.2) (layer "B.Cu") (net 9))
 (segment (start 162.5 74.5) (end 162.5 76.1485) (width 0.2) (layer "B.Cu") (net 9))
 (segment (start 145.2385 72.9485) (end 158.08 72.9485) (width 0.2) (layer "F.Cu") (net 6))
 (segment (start 143.75 71.46) (end 145.2385 72.9485) (width 0.2) (layer "F.Cu") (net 6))
 (segment (start 179.491 83.236) (end 178.859 83.236) (width 0.2) (layer "F.Cu") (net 16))
 (segment (start 175.437474 78.0285) (end 174.155 78.0285) (width 0.2) (layer "F.Cu") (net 16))
 (segment (start 174.155 78.0285) (end 172.8715 78.0285) (width 0.2) (layer "F.Cu") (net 16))
 (segment (start 176.073 78.664026) (end 175.437474 78.0285) (width 0.2) (layer "F.Cu") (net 16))
 (segment (start 176.073 79.818) (end 176.073 78.664026) (width 0.2) (layer "F.Cu") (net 16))
 (segment (start 178.859 83.236) (end 178.859 82.604) (width 0.2) (layer "F.Cu") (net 16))
 (segment (start 178.859 82.604) (end 176.073 79.818) (width 0.2) (layer "F.Cu") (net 16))
 (segment (start 180.06 83.805) (end 179.491 83.236) (width 0.2) (layer "F.Cu") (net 16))
 (segment (start 166.3 83.9) (end 166.324265 83.924265) (width 0.2) (layer "F.Cu") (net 11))
 (segment (start 176.6 82.2) (end 176.4 82) (width 0.2) (layer "F.Cu") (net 11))
 (segment (start 158.08 85.034874) (end 159.214874 83.9) (width 0.2) (layer "F.Cu") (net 11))
 (segment (start 159.214874 83.9) (end 166.3 83.9) (width 0.2) (layer "F.Cu") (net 11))
 (segment (start 176.4 82) (end 172 82) (width 0.2) (layer "F.Cu") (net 11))
 (segment (start 158.08 85.6485) (end 158.08 85.034874) (width 0.2) (layer "F.Cu") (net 11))
 (segment (start 172 82) (end 171.1 82.9) (width 0.2) (layer "F.Cu") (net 11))
 (segment (start 179.165 81.265) (end 180.06 81.265) (width 0.2) (layer "F.Cu") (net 11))
 (segment (start 177.7 79.8) (end 179.165 81.265) (width 0.2) (layer "F.Cu") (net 11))
 (via (at 166.324265 83.924265) (size 0.6) (drill 0.3) (layers "F.Cu" "B.Cu") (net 11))
 (via (at 177.7 79.8) (size 0.6) (drill 0.3) (layers "F.Cu" "B.Cu") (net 11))
 (via (at 171.1 82.9) (size 0.6) (drill 0.3) (layers "F.Cu" "B.Cu") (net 11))
 (via (at 176.6 82.2) (size 0.6) (drill 0.3) (layers "F.Cu" "B.Cu") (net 11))
 (segment (start 166.324265 83.924265) (end 170.075735 83.924265) (width 0.2) (layer "B.Cu") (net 11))
 (segment (start 177.7 81.1) (end 177.7 79.8) (width 0.2) (layer "B.Cu") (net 11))
 (segment (start 170.075735 83.924265) (end 171.1 82.9) (width 0.2) (layer "B.Cu") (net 11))
 (segment (start 176.6 82.2) (end 177.7 81.1) (width 0.2) (layer "B.Cu") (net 11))
 (segment (start 178.859 81.5261) (end 177.7339 80.401) (width 0.2) (layer "F.Cu") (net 12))
 (segment (start 172.257 78.46881) (end 172.644095 78.855905) (width 0.2) (layer "F.Cu") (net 12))
 (segment (start 179.491 81.966) (end 178.859 81.966) (width 0.2) (layer "F.Cu") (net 12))
 (segment (start 175.410626 76.9655) (end 172.87969 76.9655) (width 0.2) (layer "F.Cu") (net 12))
 (segment (start 172.644095 78.855905) (end 163.3115 88.1885) (width 0.2) (layer "F.Cu") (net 12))
 (segment (start 178.859 81.966) (end 178.859 81.5261) (width 0.2) (layer "F.Cu") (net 12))
 (segment (start 177.451057 80.401) (end 177.099 80.048943) (width 0.2) (layer "F.Cu") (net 12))
 (segment (start 172.257 77.58819) (end 172.257 78.46881) (width 0.2) (layer "F.Cu") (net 12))
 (segment (start 176.474 78.949) (end 176.474 78.028874) (width 0.2) (layer "F.Cu") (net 12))
 (segment (start 177.099 79.574) (end 176.474 78.949) (width 0.2) (layer "F.Cu") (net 12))
 (segment (start 163.3115 88.1885) (end 158.08 88.1885) (width 0.2) (layer "F.Cu") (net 12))
 (segment (start 172.87969 76.9655) (end 172.257 77.58819) (width 0.2) (layer "F.Cu") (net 12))
 (segment (start 177.7339 80.401) (end 177.451057 80.401) (width 0.2) (layer "F.Cu") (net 12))
 (segment (start 176.474 78.028874) (end 175.410626 76.9655) (width 0.2) (layer "F.Cu") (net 12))
 (segment (start 177.099 80.048943) (end 177.099 79.574) (width 0.2) (layer "F.Cu") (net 12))
 (segment (start 180.06 82.535) (end 179.491 81.966) (width 0.2) (layer "F.Cu") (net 12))
 (segment (start 158.08 78.0285) (end 145.2385 78.0285) (width 0.2) (layer "F.Cu") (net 8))
 (segment (start 145.2385 78.0285) (end 143.75 76.54) (width 0.2) (layer "F.Cu") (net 8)))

